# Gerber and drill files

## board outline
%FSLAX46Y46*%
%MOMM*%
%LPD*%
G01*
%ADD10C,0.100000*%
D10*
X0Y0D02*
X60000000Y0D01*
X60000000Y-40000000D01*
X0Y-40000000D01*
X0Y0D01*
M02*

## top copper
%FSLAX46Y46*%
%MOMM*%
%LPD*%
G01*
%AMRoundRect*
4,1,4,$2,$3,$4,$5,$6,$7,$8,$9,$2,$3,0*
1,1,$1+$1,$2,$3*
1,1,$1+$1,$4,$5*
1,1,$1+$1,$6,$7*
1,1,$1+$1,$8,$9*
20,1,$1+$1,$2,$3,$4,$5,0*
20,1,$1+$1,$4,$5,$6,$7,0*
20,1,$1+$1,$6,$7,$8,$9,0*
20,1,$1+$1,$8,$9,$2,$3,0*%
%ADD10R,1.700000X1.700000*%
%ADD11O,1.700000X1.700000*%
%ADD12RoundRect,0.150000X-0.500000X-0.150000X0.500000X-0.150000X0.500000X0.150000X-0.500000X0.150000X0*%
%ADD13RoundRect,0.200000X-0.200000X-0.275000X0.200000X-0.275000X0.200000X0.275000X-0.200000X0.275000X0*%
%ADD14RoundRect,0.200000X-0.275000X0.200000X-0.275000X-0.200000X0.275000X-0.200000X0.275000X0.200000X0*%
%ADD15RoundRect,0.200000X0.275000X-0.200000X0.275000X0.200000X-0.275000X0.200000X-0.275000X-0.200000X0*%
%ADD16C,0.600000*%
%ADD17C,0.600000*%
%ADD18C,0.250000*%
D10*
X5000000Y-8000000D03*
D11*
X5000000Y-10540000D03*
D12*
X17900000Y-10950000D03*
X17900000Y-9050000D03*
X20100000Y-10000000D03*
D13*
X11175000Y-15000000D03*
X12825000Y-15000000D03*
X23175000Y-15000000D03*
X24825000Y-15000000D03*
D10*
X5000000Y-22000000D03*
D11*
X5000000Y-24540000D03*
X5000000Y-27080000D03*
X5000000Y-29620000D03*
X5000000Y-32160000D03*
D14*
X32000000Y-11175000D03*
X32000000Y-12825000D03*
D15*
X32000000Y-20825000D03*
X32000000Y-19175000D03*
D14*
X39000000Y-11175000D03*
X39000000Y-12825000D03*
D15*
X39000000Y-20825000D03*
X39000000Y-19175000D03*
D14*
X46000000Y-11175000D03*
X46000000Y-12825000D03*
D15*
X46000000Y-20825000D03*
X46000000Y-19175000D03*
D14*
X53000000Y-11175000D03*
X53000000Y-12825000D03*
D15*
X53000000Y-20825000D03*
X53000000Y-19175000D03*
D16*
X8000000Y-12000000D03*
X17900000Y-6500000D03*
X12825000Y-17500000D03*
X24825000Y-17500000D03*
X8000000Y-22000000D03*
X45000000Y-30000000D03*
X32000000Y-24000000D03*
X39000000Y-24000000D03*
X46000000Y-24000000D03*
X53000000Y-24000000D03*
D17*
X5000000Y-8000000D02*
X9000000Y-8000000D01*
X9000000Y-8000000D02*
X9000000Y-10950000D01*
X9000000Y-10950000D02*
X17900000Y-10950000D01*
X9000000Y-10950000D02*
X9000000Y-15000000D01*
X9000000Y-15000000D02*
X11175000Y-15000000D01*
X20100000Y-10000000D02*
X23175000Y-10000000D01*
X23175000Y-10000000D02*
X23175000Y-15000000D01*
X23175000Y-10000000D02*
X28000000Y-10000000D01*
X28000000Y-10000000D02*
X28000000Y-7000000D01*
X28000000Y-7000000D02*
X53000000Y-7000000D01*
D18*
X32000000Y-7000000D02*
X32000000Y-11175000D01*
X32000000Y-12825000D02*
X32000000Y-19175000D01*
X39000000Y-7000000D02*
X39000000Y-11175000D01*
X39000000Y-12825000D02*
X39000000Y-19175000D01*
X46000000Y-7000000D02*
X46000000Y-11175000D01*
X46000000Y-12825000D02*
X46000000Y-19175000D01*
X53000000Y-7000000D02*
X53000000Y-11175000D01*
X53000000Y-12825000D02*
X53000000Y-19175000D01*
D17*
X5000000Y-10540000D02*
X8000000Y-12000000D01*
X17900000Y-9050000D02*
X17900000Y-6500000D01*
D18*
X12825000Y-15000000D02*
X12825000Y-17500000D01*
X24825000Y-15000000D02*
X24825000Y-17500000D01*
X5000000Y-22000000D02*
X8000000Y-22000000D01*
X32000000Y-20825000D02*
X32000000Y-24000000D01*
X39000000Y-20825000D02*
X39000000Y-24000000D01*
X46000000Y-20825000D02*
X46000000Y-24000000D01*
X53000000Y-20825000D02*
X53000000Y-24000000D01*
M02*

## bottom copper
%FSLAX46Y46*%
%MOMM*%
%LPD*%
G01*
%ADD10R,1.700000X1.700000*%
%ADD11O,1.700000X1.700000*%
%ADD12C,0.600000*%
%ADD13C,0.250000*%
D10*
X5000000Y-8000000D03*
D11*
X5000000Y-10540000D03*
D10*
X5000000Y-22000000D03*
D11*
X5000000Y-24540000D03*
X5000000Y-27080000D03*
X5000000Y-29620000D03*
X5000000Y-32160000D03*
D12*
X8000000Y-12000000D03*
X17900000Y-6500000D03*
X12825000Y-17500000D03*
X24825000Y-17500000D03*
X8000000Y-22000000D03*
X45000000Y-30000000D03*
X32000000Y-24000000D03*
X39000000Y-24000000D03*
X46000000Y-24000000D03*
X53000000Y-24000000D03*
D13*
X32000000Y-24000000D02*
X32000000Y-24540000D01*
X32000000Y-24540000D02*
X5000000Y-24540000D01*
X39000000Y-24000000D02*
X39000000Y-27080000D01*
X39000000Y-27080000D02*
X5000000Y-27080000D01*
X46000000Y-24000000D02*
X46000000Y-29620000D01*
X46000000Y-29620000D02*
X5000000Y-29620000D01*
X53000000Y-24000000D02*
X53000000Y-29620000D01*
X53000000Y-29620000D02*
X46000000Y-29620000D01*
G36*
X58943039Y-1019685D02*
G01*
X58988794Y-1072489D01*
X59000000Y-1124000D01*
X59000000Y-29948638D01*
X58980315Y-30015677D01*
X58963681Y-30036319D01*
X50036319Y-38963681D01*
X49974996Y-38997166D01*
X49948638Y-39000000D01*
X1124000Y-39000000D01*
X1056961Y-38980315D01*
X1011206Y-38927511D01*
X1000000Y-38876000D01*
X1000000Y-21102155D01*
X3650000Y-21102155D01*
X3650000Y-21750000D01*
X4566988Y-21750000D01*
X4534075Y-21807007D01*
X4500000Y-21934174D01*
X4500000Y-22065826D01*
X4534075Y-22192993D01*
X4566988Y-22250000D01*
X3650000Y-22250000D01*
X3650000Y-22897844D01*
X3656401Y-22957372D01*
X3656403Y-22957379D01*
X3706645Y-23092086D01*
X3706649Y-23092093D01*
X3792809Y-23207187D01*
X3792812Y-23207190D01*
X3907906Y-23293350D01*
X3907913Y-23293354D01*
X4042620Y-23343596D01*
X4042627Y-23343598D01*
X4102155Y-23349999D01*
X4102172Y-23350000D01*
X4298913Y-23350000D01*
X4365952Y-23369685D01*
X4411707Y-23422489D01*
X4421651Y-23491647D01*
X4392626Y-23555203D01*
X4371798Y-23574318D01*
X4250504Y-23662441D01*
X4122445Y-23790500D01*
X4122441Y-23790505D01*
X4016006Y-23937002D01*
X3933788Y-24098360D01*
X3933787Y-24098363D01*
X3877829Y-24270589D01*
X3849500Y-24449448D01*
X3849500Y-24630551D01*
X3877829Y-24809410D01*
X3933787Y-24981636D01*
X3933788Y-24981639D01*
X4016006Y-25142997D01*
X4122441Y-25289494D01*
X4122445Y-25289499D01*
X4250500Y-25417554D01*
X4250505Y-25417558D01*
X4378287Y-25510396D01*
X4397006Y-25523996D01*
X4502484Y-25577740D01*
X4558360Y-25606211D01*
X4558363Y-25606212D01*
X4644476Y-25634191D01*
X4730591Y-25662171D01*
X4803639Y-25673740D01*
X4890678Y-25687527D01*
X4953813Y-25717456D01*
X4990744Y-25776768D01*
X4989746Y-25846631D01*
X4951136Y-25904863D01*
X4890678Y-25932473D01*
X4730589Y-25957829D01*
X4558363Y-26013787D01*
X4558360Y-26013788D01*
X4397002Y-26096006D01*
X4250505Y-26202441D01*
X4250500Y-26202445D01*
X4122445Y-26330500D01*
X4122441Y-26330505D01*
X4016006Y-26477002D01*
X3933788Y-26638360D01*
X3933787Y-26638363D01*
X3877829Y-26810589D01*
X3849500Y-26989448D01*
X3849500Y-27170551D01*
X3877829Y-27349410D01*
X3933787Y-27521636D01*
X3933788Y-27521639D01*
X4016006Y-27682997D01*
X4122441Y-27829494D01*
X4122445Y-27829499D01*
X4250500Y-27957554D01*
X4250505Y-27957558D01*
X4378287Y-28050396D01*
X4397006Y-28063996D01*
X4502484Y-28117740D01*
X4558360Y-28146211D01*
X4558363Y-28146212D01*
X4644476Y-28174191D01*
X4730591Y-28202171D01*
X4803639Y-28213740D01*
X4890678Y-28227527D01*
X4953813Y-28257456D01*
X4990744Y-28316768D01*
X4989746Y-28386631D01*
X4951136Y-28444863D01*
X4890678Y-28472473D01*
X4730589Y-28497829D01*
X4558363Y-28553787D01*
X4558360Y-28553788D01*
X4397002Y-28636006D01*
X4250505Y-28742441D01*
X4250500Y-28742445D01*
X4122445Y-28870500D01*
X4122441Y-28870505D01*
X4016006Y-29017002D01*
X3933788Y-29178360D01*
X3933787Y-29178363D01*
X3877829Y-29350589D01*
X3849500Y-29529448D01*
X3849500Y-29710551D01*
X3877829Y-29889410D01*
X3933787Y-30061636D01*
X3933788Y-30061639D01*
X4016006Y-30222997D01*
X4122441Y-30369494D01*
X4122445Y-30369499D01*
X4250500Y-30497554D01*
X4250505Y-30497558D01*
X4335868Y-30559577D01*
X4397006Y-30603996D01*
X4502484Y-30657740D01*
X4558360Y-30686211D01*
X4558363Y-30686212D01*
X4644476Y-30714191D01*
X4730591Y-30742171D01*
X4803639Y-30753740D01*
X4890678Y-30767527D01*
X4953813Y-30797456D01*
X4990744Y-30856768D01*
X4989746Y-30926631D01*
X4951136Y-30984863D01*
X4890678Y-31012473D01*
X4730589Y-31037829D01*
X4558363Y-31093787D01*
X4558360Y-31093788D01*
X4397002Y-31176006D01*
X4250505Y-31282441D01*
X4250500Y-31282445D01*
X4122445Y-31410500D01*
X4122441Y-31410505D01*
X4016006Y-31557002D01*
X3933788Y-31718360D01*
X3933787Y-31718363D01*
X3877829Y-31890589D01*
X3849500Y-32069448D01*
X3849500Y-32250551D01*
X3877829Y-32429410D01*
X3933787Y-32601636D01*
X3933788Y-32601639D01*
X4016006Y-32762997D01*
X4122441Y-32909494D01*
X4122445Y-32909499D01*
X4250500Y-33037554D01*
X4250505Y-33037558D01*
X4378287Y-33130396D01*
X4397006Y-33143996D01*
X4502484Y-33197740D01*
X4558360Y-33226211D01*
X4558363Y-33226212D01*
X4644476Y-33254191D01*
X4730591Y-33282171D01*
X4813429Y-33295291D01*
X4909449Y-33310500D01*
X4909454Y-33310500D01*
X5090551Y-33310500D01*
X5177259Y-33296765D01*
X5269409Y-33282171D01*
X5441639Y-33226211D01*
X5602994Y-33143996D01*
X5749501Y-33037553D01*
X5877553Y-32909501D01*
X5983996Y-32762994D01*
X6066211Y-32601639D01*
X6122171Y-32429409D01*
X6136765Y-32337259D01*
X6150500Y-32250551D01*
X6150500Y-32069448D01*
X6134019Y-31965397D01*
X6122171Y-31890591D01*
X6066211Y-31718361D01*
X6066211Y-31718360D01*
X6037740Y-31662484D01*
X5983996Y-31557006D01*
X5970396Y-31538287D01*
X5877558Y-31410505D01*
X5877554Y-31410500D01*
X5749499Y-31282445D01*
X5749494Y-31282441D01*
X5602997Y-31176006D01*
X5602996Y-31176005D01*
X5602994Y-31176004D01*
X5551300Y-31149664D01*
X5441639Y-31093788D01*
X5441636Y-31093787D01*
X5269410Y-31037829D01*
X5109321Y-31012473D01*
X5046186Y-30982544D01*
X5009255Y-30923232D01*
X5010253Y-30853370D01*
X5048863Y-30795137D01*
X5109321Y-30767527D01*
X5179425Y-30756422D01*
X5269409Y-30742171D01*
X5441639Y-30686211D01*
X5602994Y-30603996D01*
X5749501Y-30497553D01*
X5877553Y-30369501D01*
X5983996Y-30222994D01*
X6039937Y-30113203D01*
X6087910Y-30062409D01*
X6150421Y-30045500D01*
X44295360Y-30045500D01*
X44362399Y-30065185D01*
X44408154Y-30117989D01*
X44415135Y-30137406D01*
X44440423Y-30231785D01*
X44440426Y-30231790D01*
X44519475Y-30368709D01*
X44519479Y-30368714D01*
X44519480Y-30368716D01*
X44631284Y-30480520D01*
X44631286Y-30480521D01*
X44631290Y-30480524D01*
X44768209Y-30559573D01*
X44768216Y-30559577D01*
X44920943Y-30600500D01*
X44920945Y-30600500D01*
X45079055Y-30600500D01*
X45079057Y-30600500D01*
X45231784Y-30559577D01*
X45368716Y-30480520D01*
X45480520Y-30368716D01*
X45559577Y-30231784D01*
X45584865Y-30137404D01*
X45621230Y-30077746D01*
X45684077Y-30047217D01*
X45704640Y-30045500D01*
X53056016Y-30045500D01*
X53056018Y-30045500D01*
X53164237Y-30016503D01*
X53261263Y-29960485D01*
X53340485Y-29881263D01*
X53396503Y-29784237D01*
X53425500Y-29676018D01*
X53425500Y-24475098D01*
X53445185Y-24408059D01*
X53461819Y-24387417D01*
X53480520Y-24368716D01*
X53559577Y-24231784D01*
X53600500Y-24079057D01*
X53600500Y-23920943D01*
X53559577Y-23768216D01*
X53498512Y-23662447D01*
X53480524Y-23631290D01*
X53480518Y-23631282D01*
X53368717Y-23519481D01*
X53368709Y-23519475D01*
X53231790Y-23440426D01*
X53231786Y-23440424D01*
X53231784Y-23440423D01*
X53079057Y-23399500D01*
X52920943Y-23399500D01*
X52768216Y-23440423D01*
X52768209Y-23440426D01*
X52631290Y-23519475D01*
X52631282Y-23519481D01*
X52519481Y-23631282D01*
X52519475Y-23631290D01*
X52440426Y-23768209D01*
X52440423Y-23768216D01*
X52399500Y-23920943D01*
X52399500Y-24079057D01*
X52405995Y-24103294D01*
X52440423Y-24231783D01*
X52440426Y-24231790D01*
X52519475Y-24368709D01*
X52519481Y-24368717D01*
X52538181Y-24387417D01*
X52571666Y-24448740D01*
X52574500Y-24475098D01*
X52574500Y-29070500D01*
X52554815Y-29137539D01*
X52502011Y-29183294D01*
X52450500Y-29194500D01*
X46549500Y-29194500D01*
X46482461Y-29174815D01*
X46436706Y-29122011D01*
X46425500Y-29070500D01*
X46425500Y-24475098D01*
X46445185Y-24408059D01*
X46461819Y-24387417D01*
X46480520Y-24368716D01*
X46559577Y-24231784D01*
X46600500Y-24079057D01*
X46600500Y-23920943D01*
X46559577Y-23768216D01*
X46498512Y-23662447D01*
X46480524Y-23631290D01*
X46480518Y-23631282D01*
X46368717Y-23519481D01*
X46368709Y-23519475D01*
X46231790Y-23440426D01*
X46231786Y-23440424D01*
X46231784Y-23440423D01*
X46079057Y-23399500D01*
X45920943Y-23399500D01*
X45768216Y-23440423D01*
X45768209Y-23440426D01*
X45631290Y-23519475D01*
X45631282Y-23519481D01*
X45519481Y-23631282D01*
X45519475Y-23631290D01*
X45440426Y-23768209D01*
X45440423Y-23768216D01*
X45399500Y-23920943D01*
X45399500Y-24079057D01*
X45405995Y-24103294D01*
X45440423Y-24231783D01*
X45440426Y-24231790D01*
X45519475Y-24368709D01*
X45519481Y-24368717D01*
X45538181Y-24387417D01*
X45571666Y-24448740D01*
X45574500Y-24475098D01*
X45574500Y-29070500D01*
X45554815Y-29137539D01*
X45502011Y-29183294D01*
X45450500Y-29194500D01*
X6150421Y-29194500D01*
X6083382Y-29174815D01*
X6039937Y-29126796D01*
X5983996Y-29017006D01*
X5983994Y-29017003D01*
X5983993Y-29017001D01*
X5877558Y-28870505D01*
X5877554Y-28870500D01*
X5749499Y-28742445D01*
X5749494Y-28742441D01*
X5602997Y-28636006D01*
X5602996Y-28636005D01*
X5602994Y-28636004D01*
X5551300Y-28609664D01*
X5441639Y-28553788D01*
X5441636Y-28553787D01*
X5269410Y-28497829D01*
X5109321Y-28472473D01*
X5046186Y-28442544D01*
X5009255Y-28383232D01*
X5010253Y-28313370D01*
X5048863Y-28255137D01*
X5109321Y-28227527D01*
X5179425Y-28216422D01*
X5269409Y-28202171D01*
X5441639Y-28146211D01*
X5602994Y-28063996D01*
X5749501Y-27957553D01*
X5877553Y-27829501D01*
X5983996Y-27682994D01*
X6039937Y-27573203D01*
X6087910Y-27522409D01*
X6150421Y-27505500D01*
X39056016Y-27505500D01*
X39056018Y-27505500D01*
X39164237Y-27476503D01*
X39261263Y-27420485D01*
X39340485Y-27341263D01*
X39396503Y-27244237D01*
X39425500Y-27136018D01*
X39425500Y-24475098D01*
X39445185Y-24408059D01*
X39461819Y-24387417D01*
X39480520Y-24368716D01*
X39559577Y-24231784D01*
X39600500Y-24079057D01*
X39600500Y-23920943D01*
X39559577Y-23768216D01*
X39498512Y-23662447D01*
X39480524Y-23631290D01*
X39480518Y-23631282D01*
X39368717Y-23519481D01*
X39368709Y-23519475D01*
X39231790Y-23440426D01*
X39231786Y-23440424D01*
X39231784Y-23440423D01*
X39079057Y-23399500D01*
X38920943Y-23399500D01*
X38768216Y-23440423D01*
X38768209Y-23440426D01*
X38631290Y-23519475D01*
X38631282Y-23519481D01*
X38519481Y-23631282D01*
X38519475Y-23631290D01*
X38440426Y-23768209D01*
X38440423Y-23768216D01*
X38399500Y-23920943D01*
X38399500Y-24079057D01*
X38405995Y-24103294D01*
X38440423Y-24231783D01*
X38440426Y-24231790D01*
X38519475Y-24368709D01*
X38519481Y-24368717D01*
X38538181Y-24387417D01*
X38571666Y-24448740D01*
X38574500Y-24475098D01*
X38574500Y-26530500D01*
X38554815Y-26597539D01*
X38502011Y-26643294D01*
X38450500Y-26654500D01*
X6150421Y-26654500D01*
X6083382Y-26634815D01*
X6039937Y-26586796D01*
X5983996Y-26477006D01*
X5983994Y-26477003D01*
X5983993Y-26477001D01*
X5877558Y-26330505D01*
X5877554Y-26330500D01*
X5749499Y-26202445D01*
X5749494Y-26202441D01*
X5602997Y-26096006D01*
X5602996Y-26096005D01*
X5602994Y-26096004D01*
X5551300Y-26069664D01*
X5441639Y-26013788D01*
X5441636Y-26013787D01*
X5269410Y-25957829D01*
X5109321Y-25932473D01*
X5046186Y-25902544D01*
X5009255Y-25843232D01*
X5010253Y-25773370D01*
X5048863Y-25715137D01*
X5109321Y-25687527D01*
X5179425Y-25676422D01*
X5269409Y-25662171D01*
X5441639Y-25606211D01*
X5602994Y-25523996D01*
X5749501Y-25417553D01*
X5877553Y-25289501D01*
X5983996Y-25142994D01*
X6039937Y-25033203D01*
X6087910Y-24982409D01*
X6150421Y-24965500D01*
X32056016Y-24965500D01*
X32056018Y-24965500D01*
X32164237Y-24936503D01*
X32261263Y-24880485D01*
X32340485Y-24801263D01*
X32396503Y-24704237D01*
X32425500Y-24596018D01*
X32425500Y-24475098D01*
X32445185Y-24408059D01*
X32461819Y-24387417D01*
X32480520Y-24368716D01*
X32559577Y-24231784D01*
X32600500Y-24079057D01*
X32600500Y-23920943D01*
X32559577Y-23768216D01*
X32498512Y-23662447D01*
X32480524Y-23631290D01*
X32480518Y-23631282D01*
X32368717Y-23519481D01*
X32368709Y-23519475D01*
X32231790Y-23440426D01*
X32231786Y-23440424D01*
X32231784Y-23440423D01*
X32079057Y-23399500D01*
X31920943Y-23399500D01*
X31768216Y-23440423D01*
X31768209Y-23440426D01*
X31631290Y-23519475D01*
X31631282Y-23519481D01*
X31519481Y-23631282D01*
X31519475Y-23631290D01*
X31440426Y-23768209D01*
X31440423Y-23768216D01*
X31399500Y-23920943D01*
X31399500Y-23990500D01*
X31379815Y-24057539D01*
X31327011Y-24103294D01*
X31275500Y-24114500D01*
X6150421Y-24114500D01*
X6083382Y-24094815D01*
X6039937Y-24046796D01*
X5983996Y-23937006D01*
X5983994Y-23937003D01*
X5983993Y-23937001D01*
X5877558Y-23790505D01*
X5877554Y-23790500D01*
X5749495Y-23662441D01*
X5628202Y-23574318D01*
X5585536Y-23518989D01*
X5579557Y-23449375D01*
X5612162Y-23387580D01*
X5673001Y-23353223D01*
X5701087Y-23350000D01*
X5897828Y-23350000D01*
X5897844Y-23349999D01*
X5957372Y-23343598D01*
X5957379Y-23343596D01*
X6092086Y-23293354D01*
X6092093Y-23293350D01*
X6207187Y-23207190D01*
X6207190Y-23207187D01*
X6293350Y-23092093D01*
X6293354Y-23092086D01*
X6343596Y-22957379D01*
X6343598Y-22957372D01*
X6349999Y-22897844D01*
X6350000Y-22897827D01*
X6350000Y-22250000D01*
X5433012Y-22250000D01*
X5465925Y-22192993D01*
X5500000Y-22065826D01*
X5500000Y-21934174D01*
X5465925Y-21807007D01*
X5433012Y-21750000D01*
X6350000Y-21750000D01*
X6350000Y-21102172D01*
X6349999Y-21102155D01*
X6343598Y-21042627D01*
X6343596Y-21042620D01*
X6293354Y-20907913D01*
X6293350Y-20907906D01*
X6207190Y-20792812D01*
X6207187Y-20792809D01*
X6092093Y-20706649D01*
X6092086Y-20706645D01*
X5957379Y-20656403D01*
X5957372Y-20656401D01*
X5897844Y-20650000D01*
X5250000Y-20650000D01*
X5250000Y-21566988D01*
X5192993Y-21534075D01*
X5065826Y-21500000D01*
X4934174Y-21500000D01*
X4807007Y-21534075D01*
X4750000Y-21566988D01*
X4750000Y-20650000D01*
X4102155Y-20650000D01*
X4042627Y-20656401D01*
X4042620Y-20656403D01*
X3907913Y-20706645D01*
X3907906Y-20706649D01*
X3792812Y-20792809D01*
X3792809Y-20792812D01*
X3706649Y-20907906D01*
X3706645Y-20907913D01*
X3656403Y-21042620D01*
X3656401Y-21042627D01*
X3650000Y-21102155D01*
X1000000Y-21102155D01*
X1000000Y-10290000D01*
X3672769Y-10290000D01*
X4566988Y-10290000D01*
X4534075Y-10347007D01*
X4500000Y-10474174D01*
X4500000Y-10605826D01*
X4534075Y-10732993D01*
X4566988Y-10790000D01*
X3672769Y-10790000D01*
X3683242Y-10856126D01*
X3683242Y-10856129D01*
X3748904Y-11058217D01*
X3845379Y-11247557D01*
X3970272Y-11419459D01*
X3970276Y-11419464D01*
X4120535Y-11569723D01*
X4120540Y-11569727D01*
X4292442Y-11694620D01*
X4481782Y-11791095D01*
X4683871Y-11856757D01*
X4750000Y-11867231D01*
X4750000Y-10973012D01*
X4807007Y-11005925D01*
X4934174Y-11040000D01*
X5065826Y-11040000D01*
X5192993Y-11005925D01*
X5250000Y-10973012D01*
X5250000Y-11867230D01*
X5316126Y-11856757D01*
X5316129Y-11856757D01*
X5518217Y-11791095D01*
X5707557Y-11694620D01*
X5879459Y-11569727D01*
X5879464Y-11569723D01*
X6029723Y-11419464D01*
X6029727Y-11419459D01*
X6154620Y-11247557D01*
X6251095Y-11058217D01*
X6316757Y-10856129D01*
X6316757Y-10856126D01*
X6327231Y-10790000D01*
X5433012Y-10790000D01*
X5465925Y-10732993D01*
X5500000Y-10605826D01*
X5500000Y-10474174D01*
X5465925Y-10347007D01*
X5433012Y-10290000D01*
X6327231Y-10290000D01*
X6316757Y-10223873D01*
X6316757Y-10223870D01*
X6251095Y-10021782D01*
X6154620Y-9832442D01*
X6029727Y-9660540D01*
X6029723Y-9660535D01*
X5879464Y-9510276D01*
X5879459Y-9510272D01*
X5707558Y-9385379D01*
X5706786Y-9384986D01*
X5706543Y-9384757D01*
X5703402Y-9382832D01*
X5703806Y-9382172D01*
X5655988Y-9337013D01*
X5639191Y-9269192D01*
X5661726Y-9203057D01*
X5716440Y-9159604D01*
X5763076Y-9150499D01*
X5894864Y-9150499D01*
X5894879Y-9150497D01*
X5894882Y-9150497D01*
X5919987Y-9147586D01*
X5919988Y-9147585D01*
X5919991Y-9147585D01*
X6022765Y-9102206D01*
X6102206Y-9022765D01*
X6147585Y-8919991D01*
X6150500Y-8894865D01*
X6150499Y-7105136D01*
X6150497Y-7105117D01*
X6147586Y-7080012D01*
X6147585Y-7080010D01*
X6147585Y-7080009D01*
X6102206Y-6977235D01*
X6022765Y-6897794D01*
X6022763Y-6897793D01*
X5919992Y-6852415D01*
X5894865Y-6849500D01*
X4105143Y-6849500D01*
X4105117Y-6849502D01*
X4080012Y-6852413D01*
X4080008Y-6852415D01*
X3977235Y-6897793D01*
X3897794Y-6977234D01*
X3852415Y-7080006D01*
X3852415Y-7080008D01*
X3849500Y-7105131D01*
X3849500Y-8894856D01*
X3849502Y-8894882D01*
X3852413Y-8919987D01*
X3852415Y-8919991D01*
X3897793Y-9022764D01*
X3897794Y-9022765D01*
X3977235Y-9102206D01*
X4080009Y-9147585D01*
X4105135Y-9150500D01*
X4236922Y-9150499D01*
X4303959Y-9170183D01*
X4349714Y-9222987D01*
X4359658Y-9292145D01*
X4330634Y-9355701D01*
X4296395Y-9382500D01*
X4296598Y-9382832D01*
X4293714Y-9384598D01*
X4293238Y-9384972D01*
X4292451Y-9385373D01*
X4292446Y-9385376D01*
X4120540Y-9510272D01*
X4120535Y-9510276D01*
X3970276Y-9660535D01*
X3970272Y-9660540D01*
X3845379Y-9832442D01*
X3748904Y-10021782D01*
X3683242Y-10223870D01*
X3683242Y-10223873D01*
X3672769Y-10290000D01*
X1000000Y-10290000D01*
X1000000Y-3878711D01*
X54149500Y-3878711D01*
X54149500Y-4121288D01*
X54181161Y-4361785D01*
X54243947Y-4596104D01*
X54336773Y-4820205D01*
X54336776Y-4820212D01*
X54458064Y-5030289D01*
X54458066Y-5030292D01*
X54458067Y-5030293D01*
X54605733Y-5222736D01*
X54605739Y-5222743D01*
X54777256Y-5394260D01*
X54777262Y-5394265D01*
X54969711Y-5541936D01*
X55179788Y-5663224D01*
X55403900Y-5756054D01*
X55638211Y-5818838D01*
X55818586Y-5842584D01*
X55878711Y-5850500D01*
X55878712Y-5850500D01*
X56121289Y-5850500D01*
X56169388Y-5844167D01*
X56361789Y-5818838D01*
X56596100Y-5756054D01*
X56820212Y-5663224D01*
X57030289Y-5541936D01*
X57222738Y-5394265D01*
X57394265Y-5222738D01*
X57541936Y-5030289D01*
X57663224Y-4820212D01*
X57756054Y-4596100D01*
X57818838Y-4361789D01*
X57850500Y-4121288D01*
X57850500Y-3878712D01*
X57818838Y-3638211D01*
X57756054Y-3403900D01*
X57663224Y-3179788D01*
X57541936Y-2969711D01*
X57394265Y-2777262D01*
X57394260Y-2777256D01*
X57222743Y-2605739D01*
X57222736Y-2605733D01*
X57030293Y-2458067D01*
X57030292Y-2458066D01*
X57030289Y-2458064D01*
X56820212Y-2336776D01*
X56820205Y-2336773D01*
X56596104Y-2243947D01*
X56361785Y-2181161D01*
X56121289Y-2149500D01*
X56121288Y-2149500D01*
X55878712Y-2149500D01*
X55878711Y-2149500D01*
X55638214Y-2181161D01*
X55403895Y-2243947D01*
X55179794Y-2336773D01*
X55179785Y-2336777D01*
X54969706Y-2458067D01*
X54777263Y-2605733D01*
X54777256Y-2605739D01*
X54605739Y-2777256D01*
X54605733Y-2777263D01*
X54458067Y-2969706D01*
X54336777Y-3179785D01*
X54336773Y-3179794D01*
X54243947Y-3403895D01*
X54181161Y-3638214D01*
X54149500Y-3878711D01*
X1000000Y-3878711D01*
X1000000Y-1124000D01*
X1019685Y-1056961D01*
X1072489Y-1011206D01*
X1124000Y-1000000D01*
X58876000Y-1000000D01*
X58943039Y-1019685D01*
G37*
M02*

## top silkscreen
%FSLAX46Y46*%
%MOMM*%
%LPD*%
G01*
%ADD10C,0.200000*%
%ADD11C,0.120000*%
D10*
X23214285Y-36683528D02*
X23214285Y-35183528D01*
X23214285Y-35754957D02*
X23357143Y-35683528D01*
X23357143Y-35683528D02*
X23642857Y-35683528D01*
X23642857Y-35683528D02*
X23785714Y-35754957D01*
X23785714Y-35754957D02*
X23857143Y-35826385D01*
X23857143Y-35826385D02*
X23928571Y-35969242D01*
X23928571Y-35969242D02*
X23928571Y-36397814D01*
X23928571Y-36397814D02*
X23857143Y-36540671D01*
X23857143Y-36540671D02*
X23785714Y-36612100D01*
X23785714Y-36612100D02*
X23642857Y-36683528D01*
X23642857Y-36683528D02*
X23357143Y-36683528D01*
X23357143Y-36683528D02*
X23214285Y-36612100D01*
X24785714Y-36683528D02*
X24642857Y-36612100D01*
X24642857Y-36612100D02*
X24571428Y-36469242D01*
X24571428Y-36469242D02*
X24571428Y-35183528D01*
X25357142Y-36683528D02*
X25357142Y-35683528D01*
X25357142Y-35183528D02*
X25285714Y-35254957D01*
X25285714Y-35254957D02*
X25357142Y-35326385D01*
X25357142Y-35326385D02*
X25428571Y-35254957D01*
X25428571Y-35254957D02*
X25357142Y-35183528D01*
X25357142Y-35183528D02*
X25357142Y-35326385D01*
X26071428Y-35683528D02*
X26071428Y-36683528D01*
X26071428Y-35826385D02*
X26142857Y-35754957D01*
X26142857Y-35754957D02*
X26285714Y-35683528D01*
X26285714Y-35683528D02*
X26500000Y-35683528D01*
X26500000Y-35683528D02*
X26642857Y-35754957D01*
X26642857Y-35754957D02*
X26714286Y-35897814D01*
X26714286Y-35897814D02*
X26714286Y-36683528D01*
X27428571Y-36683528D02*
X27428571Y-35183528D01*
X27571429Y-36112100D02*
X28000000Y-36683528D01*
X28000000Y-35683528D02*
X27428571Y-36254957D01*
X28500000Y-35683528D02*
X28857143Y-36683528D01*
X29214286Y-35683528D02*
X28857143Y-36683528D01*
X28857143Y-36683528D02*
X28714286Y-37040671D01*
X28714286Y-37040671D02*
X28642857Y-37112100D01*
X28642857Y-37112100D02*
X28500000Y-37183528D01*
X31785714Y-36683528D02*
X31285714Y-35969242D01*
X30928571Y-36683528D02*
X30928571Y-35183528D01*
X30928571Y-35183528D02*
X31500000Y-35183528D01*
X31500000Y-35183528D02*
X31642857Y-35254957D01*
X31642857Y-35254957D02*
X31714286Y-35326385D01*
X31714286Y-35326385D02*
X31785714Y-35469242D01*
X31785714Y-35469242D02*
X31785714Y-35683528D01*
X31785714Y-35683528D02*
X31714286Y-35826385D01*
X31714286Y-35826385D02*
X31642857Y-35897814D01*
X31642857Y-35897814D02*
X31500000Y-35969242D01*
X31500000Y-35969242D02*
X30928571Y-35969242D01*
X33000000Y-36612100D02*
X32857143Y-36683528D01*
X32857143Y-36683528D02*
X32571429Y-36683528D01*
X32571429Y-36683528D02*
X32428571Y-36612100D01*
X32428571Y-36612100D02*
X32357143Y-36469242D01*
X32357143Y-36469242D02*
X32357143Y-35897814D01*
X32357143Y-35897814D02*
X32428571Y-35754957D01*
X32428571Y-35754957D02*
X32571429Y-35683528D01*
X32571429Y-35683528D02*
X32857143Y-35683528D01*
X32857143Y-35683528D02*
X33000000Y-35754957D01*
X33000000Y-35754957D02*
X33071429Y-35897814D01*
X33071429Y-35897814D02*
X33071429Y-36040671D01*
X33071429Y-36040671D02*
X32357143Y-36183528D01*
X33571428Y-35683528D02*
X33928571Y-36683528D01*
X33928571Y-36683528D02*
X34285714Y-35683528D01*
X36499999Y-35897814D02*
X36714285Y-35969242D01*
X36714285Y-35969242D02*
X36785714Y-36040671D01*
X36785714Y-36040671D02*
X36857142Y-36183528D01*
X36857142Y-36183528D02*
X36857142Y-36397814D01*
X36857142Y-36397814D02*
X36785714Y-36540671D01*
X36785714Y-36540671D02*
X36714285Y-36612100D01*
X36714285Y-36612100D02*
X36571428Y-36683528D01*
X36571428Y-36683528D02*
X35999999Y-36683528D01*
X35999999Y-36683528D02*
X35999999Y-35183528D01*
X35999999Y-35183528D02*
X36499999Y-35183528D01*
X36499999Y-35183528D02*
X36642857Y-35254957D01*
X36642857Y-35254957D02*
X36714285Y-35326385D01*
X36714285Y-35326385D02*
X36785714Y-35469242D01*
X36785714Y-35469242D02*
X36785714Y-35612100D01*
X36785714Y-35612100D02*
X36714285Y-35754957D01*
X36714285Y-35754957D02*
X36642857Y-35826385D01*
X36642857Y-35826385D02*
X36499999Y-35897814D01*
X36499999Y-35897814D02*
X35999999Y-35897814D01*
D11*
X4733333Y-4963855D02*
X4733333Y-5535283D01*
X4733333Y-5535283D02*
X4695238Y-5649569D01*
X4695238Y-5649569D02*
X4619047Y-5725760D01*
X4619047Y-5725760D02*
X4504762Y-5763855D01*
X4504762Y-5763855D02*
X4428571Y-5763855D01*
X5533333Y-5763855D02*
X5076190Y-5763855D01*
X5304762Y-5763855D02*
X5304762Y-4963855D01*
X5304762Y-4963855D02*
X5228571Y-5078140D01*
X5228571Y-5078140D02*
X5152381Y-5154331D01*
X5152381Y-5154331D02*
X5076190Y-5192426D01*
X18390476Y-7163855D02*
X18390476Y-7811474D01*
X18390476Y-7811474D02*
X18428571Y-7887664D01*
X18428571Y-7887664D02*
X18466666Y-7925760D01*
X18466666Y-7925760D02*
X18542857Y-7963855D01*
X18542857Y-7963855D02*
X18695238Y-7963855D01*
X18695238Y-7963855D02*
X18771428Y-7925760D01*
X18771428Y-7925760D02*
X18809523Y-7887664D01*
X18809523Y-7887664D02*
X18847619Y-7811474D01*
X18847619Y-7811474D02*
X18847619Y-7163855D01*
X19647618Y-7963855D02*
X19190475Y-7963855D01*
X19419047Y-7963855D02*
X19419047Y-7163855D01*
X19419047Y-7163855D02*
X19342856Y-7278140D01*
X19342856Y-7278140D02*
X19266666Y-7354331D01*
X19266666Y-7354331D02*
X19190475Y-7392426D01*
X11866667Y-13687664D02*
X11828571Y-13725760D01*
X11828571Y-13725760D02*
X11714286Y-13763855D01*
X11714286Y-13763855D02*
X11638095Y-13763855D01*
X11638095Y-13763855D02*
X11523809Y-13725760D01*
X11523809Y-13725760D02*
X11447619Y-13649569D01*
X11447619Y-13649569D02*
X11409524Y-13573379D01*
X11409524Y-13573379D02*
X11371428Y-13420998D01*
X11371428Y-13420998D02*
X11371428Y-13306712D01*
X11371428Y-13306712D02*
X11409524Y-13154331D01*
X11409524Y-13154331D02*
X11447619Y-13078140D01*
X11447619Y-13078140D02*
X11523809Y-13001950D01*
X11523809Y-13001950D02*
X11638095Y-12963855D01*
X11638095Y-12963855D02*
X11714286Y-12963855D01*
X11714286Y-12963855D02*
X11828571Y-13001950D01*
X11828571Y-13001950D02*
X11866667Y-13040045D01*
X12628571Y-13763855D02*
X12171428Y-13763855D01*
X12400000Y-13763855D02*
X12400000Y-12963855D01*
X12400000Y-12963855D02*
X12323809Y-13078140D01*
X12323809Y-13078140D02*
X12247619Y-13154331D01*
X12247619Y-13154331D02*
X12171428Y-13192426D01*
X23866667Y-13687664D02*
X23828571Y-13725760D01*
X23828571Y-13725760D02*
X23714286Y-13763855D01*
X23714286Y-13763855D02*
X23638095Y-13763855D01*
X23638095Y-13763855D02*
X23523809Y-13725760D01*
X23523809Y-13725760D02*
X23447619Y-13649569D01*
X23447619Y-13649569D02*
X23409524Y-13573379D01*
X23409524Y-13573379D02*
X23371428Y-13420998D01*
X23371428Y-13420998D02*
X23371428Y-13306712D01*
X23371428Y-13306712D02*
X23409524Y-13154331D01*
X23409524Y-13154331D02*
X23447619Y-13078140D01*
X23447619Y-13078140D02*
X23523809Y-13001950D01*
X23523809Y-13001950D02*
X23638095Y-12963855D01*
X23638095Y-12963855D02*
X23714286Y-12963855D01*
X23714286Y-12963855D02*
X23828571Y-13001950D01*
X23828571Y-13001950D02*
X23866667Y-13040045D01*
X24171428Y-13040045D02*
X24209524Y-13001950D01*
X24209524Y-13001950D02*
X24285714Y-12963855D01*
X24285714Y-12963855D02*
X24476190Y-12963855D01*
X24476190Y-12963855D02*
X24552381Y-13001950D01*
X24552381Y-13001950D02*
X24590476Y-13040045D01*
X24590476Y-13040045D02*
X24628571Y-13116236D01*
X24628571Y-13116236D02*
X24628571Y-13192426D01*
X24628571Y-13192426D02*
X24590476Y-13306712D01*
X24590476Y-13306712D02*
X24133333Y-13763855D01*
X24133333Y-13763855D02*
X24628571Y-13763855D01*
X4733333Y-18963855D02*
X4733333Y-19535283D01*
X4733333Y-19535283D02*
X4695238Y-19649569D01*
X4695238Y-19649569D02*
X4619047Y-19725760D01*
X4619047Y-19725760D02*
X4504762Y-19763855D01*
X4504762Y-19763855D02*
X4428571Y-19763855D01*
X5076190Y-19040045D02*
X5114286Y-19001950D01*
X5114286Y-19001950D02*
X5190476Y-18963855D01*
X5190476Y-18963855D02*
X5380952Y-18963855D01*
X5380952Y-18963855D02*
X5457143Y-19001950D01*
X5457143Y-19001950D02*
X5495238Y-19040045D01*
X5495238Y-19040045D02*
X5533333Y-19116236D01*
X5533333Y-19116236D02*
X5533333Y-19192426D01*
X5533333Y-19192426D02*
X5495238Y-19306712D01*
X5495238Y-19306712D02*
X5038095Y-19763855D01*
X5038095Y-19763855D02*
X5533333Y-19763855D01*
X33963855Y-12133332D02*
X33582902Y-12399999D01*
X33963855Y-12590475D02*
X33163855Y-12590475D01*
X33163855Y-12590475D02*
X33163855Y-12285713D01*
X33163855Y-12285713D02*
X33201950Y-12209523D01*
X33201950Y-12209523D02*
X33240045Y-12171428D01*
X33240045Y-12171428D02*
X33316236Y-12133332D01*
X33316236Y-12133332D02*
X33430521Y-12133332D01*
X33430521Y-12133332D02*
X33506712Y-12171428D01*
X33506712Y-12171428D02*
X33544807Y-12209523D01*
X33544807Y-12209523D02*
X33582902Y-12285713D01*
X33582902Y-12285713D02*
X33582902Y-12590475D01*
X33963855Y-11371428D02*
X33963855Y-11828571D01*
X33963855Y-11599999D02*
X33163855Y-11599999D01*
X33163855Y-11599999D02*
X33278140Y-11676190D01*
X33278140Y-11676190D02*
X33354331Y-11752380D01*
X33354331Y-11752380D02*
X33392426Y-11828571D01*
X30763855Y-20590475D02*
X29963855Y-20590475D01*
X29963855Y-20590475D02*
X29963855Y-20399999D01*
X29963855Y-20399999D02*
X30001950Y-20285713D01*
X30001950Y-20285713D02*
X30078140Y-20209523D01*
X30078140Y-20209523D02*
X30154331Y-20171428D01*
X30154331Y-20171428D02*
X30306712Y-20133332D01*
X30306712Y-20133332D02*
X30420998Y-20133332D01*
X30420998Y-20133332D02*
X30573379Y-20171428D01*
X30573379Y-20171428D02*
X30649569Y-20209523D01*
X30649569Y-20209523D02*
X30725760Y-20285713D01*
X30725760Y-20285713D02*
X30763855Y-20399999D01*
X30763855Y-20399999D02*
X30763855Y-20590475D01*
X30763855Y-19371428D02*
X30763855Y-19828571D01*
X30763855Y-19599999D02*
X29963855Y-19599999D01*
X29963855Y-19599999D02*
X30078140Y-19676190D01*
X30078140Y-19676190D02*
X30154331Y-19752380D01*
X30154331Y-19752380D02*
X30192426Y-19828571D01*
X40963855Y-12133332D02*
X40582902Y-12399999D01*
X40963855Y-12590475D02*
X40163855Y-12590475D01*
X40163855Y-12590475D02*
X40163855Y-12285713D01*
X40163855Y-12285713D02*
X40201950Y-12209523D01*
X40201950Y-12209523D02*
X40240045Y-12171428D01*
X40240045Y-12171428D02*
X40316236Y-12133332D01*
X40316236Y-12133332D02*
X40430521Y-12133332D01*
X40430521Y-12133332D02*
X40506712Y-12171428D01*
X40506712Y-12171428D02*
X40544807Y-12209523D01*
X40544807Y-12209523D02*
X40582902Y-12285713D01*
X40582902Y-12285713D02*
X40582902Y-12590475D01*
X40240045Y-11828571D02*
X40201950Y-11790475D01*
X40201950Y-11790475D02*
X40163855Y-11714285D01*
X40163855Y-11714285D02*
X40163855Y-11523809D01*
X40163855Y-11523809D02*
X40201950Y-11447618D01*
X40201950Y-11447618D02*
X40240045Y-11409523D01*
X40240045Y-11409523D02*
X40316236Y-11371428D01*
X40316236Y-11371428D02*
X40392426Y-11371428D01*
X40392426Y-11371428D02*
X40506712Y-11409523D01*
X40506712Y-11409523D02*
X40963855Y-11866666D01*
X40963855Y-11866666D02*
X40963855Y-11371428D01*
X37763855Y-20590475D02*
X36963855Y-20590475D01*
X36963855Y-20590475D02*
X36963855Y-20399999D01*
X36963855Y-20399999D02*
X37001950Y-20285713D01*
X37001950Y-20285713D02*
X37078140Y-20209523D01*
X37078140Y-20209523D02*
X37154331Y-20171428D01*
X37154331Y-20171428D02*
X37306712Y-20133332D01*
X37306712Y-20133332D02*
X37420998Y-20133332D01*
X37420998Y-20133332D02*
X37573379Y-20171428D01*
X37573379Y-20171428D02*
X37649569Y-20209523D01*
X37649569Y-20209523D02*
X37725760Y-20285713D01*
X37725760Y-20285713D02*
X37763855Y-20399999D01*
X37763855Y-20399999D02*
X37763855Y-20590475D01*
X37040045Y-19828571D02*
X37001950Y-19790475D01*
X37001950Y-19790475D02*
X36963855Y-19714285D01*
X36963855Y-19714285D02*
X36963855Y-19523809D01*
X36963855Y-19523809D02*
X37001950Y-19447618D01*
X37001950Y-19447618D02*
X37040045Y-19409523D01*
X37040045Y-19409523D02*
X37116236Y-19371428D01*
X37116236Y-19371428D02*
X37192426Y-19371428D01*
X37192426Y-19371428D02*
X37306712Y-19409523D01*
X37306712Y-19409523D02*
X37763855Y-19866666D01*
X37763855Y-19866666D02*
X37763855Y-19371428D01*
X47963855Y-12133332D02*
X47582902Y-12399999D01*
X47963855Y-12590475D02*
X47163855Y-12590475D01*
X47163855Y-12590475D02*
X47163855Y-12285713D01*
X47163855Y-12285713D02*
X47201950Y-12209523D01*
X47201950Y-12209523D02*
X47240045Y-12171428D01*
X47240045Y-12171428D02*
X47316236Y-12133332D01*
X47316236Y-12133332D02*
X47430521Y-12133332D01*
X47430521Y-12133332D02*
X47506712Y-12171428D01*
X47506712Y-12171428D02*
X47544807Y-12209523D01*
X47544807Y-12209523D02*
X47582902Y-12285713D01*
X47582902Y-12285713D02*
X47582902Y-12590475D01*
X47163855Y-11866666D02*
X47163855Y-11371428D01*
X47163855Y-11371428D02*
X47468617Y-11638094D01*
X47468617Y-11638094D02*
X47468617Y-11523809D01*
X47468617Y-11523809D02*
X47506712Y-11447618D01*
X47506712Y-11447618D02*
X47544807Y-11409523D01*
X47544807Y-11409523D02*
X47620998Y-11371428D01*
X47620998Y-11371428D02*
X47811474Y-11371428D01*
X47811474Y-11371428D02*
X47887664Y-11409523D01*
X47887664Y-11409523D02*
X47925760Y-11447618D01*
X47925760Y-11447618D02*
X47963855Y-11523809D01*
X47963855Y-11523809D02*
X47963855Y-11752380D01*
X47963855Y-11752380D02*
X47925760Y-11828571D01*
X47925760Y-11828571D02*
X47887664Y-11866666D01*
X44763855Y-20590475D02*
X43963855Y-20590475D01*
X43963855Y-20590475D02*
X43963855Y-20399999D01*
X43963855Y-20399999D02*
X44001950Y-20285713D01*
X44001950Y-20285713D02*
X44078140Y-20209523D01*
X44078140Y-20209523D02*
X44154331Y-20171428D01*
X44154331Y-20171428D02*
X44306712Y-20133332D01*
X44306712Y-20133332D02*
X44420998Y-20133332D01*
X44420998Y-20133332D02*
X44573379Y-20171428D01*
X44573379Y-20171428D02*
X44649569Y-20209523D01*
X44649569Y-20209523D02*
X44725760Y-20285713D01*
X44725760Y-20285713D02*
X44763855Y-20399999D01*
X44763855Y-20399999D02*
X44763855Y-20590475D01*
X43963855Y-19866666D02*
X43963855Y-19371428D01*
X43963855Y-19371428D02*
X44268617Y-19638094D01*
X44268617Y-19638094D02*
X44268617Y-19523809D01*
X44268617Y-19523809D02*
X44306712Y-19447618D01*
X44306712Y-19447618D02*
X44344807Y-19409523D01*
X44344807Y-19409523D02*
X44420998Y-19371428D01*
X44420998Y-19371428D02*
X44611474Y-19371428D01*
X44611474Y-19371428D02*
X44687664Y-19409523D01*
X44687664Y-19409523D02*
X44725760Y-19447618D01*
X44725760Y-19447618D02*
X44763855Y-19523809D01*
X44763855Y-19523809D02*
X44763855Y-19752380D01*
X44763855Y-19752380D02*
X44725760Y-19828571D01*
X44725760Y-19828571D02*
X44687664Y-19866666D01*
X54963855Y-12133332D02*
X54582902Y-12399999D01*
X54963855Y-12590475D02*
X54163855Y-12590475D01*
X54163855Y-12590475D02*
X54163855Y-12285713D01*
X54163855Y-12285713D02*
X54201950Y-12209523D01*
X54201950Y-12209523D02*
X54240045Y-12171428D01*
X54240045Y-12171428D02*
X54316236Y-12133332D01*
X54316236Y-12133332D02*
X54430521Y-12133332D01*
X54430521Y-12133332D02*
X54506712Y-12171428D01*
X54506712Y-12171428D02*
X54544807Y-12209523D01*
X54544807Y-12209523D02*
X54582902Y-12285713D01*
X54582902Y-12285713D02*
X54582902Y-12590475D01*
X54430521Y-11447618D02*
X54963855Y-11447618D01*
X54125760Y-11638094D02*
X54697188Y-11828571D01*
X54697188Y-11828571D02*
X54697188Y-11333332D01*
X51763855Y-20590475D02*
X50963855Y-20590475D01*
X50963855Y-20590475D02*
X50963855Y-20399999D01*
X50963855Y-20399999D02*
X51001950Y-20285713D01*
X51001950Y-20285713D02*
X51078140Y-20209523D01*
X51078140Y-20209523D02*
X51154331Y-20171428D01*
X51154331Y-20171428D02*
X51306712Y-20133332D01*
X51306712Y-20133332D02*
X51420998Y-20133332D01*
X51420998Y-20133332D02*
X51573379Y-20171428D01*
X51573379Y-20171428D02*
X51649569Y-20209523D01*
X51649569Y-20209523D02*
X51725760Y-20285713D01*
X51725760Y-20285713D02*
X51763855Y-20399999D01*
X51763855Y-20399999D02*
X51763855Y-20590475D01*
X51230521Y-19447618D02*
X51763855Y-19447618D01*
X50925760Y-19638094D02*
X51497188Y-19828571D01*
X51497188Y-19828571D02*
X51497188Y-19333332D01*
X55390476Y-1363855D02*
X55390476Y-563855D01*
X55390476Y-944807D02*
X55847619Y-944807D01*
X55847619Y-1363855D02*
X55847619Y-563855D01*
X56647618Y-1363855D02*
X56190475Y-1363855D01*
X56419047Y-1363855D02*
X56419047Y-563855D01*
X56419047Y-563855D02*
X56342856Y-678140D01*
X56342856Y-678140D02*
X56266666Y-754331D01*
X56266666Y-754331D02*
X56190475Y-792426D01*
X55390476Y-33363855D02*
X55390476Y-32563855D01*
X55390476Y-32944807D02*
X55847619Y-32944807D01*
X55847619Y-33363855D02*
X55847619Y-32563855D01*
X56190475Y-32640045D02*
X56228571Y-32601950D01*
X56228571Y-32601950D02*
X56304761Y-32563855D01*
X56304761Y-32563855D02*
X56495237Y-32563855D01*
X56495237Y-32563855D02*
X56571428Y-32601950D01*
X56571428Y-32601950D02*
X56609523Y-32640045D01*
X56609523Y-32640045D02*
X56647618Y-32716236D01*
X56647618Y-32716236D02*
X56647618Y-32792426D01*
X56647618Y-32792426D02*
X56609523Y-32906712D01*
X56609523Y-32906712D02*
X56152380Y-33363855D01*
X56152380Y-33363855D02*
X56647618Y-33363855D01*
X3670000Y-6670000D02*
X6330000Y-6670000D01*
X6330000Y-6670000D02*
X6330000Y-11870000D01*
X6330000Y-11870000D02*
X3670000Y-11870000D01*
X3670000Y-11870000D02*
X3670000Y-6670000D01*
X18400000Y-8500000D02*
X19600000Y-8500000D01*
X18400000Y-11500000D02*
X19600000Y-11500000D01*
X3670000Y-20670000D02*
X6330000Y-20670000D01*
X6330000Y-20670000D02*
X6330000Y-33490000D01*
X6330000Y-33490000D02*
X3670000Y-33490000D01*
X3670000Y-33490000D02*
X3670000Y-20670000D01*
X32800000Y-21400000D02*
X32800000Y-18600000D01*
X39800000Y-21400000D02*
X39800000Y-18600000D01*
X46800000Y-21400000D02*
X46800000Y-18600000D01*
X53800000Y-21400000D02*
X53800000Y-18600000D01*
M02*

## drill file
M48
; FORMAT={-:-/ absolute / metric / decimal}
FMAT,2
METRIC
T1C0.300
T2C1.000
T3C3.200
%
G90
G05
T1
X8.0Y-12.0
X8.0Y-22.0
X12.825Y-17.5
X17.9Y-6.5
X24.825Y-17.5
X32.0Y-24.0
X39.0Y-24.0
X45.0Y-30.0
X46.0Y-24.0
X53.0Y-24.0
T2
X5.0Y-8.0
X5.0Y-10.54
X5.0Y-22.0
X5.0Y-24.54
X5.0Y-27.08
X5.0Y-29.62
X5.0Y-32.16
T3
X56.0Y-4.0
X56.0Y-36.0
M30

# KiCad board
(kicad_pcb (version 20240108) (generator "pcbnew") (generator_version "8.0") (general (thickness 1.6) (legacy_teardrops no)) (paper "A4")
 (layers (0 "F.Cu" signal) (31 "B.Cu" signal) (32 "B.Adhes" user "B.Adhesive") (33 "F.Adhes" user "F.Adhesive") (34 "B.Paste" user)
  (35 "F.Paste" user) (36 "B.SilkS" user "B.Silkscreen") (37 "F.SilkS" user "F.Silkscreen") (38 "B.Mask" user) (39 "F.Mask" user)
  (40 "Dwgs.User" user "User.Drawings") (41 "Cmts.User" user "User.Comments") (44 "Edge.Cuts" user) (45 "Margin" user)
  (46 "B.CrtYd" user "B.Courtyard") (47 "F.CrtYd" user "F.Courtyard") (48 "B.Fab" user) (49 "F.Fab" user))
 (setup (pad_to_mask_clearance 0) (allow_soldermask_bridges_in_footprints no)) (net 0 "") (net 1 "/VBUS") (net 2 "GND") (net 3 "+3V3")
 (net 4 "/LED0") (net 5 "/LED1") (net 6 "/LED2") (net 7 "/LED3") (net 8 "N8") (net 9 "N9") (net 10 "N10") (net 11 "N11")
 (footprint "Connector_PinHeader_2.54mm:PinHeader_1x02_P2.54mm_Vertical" (layer "F.Cu") (at 5 8)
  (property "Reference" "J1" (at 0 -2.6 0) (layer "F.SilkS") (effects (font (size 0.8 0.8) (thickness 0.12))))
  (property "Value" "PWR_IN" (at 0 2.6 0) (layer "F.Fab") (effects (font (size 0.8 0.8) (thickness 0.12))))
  (fp_line (start -1.33 -1.33) (end 1.33 -1.33) (stroke (width 0.12) (type solid)) (layer "F.SilkS"))
  (fp_line (start 1.33 -1.33) (end 1.33 3.87) (stroke (width 0.12) (type solid)) (layer "F.SilkS"))
  (fp_line (start 1.33 3.87) (end -1.33 3.87) (stroke (width 0.12) (type solid)) (layer "F.SilkS"))
  (fp_line (start -1.33 3.87) (end -1.33 -1.33) (stroke (width 0.12) (type solid)) (layer "F.SilkS"))
  (pad "1" thru_hole rect (at 0 0) (size 1.7 1.7) (drill 1) (layers "*.Cu" "*.Mask") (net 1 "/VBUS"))
  (pad "2" thru_hole oval (at 0 2.54) (size 1.7 1.7) (drill 1) (layers "*.Cu" "*.Mask") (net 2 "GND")))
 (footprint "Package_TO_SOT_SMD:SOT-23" (layer "F.Cu") (at 19 10)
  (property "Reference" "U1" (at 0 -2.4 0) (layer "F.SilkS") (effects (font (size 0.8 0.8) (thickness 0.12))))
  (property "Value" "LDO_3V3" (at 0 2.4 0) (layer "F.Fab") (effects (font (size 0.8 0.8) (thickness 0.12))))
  (fp_line (start -0.6 -1.5) (end 0.6 -1.5) (stroke (width 0.12) (type solid)) (layer "F.SilkS"))
  (fp_line (start -0.6 1.5) (end 0.6 1.5) (stroke (width 0.12) (type solid)) (layer "F.SilkS"))
  (pad "1" smd roundrect (at -1.1 0.95) (size 1.3 0.6) (layers "F.Cu" "F.Paste" "F.Mask") (roundrect_rratio 0.25) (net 1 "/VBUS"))
  (pad "2" smd roundrect (at -1.1 -0.95) (size 1.3 0.6) (layers "F.Cu" "F.Paste" "F.Mask") (roundrect_rratio 0.25) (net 2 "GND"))
  (pad "3" smd roundrect (at 1.1 0) (size 1.3 0.6) (layers "F.Cu" "F.Paste" "F.Mask") (roundrect_rratio 0.25) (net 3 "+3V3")))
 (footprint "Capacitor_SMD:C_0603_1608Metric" (layer "F.Cu") (at 12 15)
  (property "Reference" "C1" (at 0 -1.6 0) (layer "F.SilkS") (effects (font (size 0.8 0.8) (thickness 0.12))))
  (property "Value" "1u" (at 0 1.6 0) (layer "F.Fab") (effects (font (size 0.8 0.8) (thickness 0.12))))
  (pad "1" smd roundrect (at -0.825 0) (size 0.8 0.95) (layers "F.Cu" "F.Paste" "F.Mask") (roundrect_rratio 0.25) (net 1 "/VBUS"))
  (pad "2" smd roundrect (at 0.825 0) (size 0.8 0.95) (layers "F.Cu" "F.Paste" "F.Mask") (roundrect_rratio 0.25) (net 2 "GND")))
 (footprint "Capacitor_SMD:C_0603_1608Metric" (layer "F.Cu") (at 24 15)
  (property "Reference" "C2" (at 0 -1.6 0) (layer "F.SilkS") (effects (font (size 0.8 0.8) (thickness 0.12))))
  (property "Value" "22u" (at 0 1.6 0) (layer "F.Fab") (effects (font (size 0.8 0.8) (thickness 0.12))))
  (pad "1" smd roundrect (at -0.825 0) (size 0.8 0.95) (layers "F.Cu" "F.Paste" "F.Mask") (roundrect_rratio 0.25) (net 3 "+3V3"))
  (pad "2" smd roundrect (at 0.825 0) (size 0.8 0.95) (layers "F.Cu" "F.Paste" "F.Mask") (roundrect_rratio 0.25) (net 2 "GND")))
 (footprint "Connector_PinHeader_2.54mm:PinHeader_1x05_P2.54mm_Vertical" (layer "F.Cu") (at 5 22)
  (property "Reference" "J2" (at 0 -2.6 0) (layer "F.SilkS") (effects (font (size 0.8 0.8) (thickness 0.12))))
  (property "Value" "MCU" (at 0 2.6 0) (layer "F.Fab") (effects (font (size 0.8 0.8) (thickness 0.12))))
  (fp_line (start -1.33 -1.33) (end 1.33 -1.33) (stroke (width 0.12) (type solid)) (layer "F.SilkS"))
  (fp_line (start 1.33 -1.33) (end 1.33 11.49) (stroke (width 0.12) (type solid)) (layer "F.SilkS"))
  (fp_line (start 1.33 11.49) (end -1.33 11.49) (stroke (width 0.12) (type solid)) (layer "F.SilkS"))
  (fp_line (start -1.33 11.49) (end -1.33 -1.33) (stroke (width 0.12) (type solid)) (layer "F.SilkS"))
  (pad "1" thru_hole rect (at 0 0) (size 1.7 1.7) (drill 1) (layers "*.Cu" "*.Mask") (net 2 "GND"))
  (pad "2" thru_hole oval (at 0 2.54) (size 1.7 1.7) (drill 1) (layers "*.Cu" "*.Mask") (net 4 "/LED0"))
  (pad "3" thru_hole oval (at 0 5.08) (size 1.7 1.7) (drill 1) (layers "*.Cu" "*.Mask") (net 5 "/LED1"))
  (pad "4" thru_hole oval (at 0 7.62) (size 1.7 1.7) (drill 1) (layers "*.Cu" "*.Mask") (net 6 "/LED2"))
  (pad "5" thru_hole oval (at 0 10.16) (size 1.7 1.7) (drill 1) (layers "*.Cu" "*.Mask") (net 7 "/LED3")))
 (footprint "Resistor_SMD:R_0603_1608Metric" (layer "F.Cu") (at 32 12 270)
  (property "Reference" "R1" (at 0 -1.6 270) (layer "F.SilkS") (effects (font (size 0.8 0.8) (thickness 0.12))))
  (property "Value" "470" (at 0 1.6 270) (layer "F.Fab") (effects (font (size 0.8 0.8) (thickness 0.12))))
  (pad "1" smd roundrect (at -0.825 0 270) (size 0.8 0.95) (layers "F.Cu" "F.Paste" "F.Mask") (roundrect_rratio 0.25) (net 3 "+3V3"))
  (pad "2" smd roundrect (at 0.825 0 270) (size 0.8 0.95) (layers "F.Cu" "F.Paste" "F.Mask") (roundrect_rratio 0.25) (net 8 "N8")))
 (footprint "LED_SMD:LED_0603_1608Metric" (layer "F.Cu") (at 32 20 90)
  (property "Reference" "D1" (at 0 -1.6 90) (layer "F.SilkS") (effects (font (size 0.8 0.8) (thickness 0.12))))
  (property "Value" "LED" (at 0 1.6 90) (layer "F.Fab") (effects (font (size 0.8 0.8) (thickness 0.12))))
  (fp_line (start -1.4 0.8) (end 1.4 0.8) (stroke (width 0.12) (type solid)) (layer "F.SilkS"))
  (pad "1" smd roundrect (at -0.825 0 90) (size 0.8 0.95) (layers "F.Cu" "F.Paste" "F.Mask") (roundrect_rratio 0.25) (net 4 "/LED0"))
  (pad "2" smd roundrect (at 0.825 0 90) (size 0.8 0.95) (layers "F.Cu" "F.Paste" "F.Mask") (roundrect_rratio 0.25) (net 8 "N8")))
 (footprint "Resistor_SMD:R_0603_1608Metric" (layer "F.Cu") (at 39 12 270)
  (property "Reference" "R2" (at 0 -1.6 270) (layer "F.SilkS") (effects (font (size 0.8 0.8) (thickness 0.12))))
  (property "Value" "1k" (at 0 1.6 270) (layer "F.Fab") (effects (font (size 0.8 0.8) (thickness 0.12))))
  (pad "1" smd roundrect (at -0.825 0 270) (size 0.8 0.95) (layers "F.Cu" "F.Paste" "F.Mask") (roundrect_rratio 0.25) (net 3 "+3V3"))
  (pad "2" smd roundrect (at 0.825 0 270) (size 0.8 0.95) (layers "F.Cu" "F.Paste" "F.Mask") (roundrect_rratio 0.25) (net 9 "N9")))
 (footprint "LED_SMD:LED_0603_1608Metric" (layer "F.Cu") (at 39 20 90)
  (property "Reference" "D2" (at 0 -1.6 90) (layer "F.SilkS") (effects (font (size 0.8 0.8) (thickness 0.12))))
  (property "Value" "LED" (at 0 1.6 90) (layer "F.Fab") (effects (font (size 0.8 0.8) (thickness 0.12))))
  (fp_line (start -1.4 0.8) (end 1.4 0.8) (stroke (width 0.12) (type solid)) (layer "F.SilkS"))
  (pad "1" smd roundrect (at -0.825 0 90) (size 0.8 0.95) (layers "F.Cu" "F.Paste" "F.Mask") (roundrect_rratio 0.25) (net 5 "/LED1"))
  (pad "2" smd roundrect (at 0.825 0 90) (size 0.8 0.95) (layers "F.Cu" "F.Paste" "F.Mask") (roundrect_rratio 0.25) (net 9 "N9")))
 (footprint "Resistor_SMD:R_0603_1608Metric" (layer "F.Cu") (at 46 12 270)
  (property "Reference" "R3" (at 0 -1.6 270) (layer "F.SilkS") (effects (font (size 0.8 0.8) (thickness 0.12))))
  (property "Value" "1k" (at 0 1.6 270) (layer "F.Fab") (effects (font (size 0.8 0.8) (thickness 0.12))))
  (pad "1" smd roundrect (at -0.825 0 270) (size 0.8 0.95) (layers "F.Cu" "F.Paste" "F.Mask") (roundrect_rratio 0.25) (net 3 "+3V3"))
  (pad "2" smd roundrect (at 0.825 0 270) (size 0.8 0.95) (layers "F.Cu" "F.Paste" "F.Mask") (roundrect_rratio 0.25) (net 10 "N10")))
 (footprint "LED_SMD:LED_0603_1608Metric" (layer "F.Cu") (at 46 20 90)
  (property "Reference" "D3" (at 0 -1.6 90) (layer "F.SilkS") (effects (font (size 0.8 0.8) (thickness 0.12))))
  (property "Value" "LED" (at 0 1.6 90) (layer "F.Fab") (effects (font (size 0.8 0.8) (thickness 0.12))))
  (fp_line (start -1.4 0.8) (end 1.4 0.8) (stroke (width 0.12) (type solid)) (layer "F.SilkS"))
  (pad "1" smd roundrect (at -0.825 0 90) (size 0.8 0.95) (layers "F.Cu" "F.Paste" "F.Mask") (roundrect_rratio 0.25) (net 6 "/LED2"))
  (pad "2" smd roundrect (at 0.825 0 90) (size 0.8 0.95) (layers "F.Cu" "F.Paste" "F.Mask") (roundrect_rratio 0.25) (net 10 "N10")))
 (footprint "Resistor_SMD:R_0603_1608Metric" (layer "F.Cu") (at 53 12 270)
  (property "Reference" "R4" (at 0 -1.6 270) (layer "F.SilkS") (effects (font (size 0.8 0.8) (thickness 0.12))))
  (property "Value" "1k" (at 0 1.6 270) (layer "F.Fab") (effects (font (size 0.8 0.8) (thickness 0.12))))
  (pad "1" smd roundrect (at -0.825 0 270) (size 0.8 0.95) (layers "F.Cu" "F.Paste" "F.Mask") (roundrect_rratio 0.25) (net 3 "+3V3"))
  (pad "2" smd roundrect (at 0.825 0 270) (size 0.8 0.95) (layers "F.Cu" "F.Paste" "F.Mask") (roundrect_rratio 0.25) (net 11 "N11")))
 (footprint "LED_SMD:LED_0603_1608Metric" (layer "F.Cu") (at 53 20 90)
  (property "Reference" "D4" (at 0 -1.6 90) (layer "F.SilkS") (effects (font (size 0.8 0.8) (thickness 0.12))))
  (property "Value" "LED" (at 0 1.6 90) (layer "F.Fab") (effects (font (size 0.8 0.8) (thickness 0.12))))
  (fp_line (start -1.4 0.8) (end 1.4 0.8) (stroke (width 0.12) (type solid)) (layer "F.SilkS"))
  (pad "1" smd roundrect (at -0.825 0 90) (size 0.8 0.95) (layers "F.Cu" "F.Paste" "F.Mask") (roundrect_rratio 0.25) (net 6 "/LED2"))
  (pad "2" smd roundrect (at 0.825 0 90) (size 0.8 0.95) (layers "F.Cu" "F.Paste" "F.Mask") (roundrect_rratio 0.25) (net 11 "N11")))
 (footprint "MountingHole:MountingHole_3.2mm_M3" (layer "F.Cu") (at 56 4)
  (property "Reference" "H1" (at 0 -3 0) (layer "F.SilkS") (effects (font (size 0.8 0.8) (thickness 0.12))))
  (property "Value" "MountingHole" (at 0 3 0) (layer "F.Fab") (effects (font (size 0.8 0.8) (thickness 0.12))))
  (pad "" np_thru_hole circle (at 0 0) (size 3.2 3.2) (drill 3.2) (layers "*.Cu" "*.Mask")))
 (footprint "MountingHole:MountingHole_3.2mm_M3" (layer "F.Cu") (at 56 36)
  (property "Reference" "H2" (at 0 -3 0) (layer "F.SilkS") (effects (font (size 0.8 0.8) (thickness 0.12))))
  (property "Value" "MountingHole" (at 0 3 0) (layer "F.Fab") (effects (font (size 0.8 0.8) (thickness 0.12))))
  (pad "" np_thru_hole circle (at 0 0) (size 3.2 3.2) (drill 3.2) (layers "*.Cu" "*.Mask")))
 (segment (start 5 8) (end 9 8) (width 0.6) (layer "F.Cu") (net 1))
 (segment (start 9 8) (end 9 10.95) (width 0.6) (layer "F.Cu") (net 1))
 (segment (start 9 10.95) (end 17.9 10.95) (width 0.6) (layer "F.Cu") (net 1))
 (segment (start 9 10.95) (end 9 15) (width 0.6) (layer "F.Cu") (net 1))
 (segment (start 9 15) (end 11.175 15) (width 0.6) (layer "F.Cu") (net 1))
 (segment (start 20.1 10) (end 23.175 10) (width 0.6) (layer "F.Cu") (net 3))
 (segment (start 23.175 10) (end 23.175 15) (width 0.6) (layer "F.Cu") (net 3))
 (segment (start 23.175 10) (end 28 10) (width 0.6) (layer "F.Cu") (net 3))
 (segment (start 28 10) (end 28 7) (width 0.6) (layer "F.Cu") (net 3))
 (segment (start 28 7) (end 53 7) (width 0.6) (layer "F.Cu") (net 3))
 (segment (start 32 7) (end 32 11.175) (width 0.25) (layer "F.Cu") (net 3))
 (segment (start 32 12.825) (end 32 19.175) (width 0.25) (layer "F.Cu") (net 8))
 (segment (start 39 7) (end 39 11.175) (width 0.25) (layer "F.Cu") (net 3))
 (segment (start 39 12.825) (end 39 19.175) (width 0.25) (layer "F.Cu") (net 9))
 (segment (start 46 7) (end 46 11.175) (width 0.25) (layer "F.Cu") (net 3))
 (segment (start 46 12.825) (end 46 19.175) (width 0.25) (layer "F.Cu") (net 10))
 (segment (start 53 7) (end 53 11.175) (width 0.25) (layer "F.Cu") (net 3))
 (segment (start 53 12.825) (end 53 19.175) (width 0.25) (layer "F.Cu") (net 11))
 (segment (start 5 10.54) (end 8 12) (width 0.6) (layer "F.Cu") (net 2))
 (via (at 8 12) (size 0.6) (drill 0.3) (layers "F.Cu" "B.Cu") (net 2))
 (segment (start 17.9 9.05) (end 17.9 6.5) (width 0.6) (layer "F.Cu") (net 2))
 (via (at 17.9 6.5) (size 0.6) (drill 0.3) (layers "F.Cu" "B.Cu") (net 2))
 (segment (start 12.825 15) (end 12.825 17.5) (width 0.25) (layer "F.Cu") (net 2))
 (via (at 12.825 17.5) (size 0.6) (drill 0.3) (layers "F.Cu" "B.Cu") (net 2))
 (segment (start 24.825 15) (end 24.825 17.5) (width 0.25) (layer "F.Cu") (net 2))
 (via (at 24.825 17.5) (size 0.6) (drill 0.3) (layers "F.Cu" "B.Cu") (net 2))
 (segment (start 5 22) (end 8 22) (width 0.25) (layer "F.Cu") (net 2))
 (via (at 8 22) (size 0.6) (drill 0.3) (layers "F.Cu" "B.Cu") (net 2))
 (via (at 45 30) (size 0.6) (drill 0.3) (layers "F.Cu" "B.Cu") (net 2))
 (segment (start 32 20.825) (end 32 24) (width 0.25) (layer "F.Cu") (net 4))
 (via (at 32 24) (size 0.6) (drill 0.3) (layers "F.Cu" "B.Cu") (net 4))
 (segment (start 32 24) (end 32 24.54) (width 0.25) (layer "B.Cu") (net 4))
 (segment (start 32 24.54) (end 5 24.54) (width 0.25) (layer "B.Cu") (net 4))
 (segment (start 39 20.825) (end 39 24) (width 0.25) (layer "F.Cu") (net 5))
 (via (at 39 24) (size 0.6) (drill 0.3) (layers "F.Cu" "B.Cu") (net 5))
 (segment (start 39 24) (end 39 27.08) (width 0.25) (layer "B.Cu") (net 5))
 (segment (start 39 27.08) (end 5 27.08) (width 0.25) (layer "B.Cu") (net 5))
 (segment (start 46 20.825) (end 46 24) (width 0.25) (layer "F.Cu") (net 6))
 (via (at 46 24) (size 0.6) (drill 0.3) (layers "F.Cu" "B.Cu") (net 6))
 (segment (start 46 24) (end 46 29.62) (width 0.25) (layer "B.Cu") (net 6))
 (segment (start 46 29.62) (end 5 29.62) (width 0.25) (layer "B.Cu") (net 6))
 (segment (start 53 20.825) (end 53 24) (width 0.25) (layer "F.Cu") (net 6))
 (via (at 53 24) (size 0.6) (drill 0.3) (layers "F.Cu" "B.Cu") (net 6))
 (segment (start 53 24) (end 53 29.62) (width 0.25) (layer "B.Cu") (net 6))
 (segment (start 53 29.62) (end 46 29.62) (width 0.25) (layer "B.Cu") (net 6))
 (gr_rect (start 0 0) (end 60 40) (stroke (width 0.1) (type default)) (fill none) (layer "Edge.Cuts"))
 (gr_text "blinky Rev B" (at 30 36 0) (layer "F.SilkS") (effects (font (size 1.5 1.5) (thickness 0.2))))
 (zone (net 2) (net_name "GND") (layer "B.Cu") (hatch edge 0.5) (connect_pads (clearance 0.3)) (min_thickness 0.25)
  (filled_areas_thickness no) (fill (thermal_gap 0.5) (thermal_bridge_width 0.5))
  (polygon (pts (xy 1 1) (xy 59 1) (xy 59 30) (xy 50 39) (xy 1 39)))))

